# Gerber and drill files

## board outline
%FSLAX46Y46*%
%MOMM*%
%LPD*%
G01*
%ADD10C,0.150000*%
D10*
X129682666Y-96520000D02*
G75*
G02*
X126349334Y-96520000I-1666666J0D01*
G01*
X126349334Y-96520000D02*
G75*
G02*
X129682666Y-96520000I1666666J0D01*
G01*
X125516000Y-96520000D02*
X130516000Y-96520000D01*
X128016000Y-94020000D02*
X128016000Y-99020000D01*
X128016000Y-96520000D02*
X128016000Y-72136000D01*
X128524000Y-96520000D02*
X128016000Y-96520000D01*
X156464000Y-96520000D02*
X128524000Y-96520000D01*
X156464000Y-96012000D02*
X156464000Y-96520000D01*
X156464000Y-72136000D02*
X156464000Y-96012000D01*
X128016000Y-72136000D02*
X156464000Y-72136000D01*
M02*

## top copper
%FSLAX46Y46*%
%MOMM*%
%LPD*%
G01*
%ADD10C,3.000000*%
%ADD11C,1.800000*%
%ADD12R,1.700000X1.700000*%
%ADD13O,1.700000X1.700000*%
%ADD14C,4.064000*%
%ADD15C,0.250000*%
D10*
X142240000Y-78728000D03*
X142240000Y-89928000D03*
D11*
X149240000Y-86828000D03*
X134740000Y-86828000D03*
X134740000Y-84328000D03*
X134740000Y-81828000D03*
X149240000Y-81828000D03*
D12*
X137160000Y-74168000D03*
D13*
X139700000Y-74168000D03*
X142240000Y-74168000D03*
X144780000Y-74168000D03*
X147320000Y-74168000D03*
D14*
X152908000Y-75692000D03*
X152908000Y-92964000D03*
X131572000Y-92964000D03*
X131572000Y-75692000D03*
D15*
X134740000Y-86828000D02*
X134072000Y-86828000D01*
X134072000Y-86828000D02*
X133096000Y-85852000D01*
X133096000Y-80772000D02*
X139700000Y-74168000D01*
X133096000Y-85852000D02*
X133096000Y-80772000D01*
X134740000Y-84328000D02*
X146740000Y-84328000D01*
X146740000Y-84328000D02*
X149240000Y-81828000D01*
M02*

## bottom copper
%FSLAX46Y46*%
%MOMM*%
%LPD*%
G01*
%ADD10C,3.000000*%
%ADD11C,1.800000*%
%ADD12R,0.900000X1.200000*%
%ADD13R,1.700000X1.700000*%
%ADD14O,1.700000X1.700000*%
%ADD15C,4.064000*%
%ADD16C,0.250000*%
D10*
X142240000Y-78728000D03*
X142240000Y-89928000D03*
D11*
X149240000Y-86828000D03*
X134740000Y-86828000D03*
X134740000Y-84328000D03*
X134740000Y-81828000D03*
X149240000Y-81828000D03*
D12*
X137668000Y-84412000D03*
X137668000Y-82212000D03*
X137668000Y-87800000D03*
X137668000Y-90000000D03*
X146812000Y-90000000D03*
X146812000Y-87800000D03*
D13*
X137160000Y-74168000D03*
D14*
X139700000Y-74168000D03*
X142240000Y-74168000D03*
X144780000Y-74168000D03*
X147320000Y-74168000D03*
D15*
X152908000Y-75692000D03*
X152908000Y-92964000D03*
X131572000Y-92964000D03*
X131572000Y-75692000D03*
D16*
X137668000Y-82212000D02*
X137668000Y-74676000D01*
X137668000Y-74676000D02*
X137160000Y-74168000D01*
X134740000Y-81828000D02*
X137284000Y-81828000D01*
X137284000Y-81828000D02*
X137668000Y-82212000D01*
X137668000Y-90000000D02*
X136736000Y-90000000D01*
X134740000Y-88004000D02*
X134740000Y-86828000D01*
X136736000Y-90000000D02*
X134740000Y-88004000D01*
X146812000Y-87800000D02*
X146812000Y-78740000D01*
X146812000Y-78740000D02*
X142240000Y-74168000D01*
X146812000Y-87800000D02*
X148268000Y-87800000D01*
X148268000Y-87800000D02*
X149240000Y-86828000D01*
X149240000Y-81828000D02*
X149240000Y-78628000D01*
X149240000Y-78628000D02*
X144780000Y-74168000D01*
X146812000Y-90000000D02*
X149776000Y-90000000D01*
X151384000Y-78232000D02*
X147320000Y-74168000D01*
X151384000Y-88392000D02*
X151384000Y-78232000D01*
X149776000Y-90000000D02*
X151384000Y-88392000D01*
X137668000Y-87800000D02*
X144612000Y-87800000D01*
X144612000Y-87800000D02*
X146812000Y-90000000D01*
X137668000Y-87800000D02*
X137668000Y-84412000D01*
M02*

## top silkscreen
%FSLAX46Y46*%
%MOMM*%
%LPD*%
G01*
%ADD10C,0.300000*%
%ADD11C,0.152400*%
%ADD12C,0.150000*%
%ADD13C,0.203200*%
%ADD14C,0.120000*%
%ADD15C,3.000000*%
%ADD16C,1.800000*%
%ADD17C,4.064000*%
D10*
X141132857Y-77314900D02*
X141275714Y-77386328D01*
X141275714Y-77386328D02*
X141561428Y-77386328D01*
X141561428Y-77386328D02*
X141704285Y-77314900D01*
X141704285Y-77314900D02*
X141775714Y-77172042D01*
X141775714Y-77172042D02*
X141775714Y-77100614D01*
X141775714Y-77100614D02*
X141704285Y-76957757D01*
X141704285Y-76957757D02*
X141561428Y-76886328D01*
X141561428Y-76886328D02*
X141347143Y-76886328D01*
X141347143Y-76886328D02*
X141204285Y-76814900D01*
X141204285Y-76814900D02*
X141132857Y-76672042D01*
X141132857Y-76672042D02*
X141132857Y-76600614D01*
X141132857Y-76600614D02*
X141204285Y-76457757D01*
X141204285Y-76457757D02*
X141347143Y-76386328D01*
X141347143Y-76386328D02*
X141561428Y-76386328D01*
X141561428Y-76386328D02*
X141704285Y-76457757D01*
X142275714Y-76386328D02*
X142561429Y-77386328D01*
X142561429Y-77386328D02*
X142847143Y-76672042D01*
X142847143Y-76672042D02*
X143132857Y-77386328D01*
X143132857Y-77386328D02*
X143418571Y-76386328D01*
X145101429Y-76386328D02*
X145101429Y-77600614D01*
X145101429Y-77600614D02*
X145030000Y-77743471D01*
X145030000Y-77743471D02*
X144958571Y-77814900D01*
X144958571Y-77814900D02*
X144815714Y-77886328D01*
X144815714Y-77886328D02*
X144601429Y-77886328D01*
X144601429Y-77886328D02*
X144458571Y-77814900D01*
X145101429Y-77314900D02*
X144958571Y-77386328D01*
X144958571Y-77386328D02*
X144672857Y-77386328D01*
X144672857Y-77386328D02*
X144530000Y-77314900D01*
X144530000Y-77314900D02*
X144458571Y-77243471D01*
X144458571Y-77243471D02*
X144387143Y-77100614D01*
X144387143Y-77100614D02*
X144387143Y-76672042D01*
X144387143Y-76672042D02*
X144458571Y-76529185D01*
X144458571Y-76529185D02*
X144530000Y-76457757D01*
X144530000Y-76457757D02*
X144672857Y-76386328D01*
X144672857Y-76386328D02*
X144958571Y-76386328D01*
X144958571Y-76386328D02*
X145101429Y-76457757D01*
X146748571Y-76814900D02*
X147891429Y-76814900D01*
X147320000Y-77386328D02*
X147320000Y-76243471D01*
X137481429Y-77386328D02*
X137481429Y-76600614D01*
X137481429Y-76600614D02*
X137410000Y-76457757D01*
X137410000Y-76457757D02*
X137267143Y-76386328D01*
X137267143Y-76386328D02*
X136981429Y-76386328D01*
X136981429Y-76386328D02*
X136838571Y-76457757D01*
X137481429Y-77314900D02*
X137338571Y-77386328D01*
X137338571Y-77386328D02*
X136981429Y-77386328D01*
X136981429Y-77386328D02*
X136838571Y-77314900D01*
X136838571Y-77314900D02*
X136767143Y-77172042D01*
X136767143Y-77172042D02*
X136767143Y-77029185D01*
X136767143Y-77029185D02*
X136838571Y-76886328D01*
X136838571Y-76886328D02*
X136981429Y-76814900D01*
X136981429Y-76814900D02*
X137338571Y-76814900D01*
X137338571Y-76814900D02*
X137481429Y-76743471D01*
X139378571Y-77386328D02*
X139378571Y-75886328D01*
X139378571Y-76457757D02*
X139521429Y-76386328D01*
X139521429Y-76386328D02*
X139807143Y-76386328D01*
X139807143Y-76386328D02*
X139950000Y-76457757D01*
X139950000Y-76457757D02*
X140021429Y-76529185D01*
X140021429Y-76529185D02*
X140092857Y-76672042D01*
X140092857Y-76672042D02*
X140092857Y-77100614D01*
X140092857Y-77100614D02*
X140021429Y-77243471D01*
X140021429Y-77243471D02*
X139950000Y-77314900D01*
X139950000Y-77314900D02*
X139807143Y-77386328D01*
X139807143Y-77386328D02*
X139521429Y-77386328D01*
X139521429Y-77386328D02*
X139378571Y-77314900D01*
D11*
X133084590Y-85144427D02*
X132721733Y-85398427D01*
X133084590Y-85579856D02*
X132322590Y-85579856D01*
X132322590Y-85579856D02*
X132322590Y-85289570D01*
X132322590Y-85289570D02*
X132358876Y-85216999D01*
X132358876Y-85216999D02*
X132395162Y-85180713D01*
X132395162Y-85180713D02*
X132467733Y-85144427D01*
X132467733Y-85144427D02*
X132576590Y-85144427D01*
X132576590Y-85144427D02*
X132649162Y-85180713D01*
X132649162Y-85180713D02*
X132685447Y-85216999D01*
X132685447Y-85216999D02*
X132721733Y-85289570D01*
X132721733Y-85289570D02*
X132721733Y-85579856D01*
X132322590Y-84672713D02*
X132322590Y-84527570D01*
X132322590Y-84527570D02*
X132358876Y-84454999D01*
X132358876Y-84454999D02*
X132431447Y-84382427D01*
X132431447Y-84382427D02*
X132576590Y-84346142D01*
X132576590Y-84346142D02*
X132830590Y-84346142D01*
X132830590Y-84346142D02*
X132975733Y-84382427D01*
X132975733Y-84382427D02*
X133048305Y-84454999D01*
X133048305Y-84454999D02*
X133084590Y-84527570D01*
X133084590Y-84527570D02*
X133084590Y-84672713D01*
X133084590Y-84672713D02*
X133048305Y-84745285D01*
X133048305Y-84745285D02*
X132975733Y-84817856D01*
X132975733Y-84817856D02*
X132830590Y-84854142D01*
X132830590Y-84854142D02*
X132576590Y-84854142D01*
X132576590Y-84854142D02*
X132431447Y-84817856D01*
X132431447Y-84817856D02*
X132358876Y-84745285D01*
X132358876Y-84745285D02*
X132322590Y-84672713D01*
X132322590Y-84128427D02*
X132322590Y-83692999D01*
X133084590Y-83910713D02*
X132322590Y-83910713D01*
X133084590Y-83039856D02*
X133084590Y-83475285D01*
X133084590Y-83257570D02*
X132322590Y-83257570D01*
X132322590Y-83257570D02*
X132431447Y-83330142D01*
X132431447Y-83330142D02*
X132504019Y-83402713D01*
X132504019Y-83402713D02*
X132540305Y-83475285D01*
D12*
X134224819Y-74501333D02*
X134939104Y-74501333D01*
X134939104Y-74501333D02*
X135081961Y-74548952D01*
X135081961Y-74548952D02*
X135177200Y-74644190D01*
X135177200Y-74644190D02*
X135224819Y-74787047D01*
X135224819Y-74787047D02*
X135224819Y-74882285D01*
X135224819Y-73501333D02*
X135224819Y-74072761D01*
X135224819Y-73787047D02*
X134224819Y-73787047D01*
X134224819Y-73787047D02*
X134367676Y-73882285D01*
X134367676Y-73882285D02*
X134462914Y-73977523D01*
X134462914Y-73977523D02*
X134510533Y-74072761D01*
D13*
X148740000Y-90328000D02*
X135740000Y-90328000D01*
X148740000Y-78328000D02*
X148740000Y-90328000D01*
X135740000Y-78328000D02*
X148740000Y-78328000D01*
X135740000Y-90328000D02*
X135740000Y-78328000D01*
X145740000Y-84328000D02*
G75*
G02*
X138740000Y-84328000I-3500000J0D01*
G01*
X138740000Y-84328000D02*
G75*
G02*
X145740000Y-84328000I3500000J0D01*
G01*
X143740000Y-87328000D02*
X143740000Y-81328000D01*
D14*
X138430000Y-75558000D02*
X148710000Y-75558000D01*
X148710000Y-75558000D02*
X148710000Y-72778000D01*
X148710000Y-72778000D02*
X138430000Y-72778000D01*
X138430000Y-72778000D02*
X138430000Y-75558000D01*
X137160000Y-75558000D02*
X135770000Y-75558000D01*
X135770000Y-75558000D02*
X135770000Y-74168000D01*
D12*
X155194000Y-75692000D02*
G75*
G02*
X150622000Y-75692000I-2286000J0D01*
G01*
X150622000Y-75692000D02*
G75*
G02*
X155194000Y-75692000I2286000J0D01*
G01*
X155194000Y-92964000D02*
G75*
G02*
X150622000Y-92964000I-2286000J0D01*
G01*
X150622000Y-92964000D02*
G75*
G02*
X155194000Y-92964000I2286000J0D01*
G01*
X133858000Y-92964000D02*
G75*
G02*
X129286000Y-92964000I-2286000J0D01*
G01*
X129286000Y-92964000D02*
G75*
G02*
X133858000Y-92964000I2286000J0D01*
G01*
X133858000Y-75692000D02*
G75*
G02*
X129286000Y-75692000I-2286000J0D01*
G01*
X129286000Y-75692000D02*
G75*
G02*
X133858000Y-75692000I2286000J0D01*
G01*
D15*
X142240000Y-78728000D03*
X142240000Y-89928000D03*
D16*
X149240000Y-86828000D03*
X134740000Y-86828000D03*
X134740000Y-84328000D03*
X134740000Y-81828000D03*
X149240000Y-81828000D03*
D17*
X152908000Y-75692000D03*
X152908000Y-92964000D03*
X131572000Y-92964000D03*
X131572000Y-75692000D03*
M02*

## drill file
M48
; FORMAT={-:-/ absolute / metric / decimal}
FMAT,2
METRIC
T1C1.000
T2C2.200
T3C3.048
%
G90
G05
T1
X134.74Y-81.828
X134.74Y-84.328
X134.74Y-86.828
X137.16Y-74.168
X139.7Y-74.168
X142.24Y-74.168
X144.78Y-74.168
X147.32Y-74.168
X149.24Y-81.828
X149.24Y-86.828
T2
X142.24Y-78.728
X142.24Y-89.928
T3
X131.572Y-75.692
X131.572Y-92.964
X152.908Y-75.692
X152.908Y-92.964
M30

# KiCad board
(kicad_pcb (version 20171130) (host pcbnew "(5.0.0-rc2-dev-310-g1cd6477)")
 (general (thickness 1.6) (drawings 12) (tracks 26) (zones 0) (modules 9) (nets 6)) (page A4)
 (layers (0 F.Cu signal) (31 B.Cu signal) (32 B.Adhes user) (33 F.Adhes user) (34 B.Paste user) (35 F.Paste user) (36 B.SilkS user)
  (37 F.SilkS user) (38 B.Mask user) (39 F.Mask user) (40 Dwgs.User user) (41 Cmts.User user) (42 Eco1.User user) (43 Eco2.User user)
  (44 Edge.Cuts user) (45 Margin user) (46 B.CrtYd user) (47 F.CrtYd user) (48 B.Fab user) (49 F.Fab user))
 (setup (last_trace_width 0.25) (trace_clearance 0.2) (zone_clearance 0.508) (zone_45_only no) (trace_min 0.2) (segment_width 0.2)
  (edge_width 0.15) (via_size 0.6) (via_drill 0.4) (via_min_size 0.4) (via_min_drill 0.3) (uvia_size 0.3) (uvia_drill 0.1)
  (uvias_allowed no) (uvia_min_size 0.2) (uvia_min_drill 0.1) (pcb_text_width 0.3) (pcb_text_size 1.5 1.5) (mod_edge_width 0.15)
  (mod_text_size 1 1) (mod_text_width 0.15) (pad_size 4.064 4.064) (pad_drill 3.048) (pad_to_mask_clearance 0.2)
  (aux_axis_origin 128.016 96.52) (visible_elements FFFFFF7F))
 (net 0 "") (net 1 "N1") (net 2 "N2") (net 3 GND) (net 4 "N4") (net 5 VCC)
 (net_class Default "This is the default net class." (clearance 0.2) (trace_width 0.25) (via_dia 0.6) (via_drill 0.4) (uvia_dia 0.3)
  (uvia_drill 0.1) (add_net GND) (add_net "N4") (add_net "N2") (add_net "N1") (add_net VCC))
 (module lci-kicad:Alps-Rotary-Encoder (layer F.Cu) (at 142.24 84.328 270)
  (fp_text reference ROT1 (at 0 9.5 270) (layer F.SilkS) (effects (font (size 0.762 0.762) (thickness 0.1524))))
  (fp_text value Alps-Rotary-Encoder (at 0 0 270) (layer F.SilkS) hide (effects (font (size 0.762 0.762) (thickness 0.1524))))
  (fp_line (start 6 -6.5) (end 6 6.5) (layer F.SilkS) (width 0.2032))
  (fp_line (start -6 -6.5) (end 6 -6.5) (layer F.SilkS) (width 0.2032))
  (fp_line (start -6 6.5) (end -6 -6.5) (layer F.SilkS) (width 0.2032))
  (fp_line (start 6 6.5) (end -6 6.5) (layer F.SilkS) (width 0.2032))
  (fp_circle (center 0 0) (end 3.5 0) (layer F.SilkS) (width 0.2032))
  (fp_line (start 3 -1.5) (end -3 -1.5) (layer F.SilkS) (width 0.2032))
  (pad "" thru_hole circle (at -5.6 0 270) (size 3 3) (drill 2.2) (layers *.Cu *.Mask F.SilkS))
  (pad "" thru_hole circle (at 5.6 0 270) (size 3 3) (drill 2.2) (layers *.Cu *.Mask F.SilkS))
  (pad 5 thru_hole circle (at 2.5 -7 270) (size 1.8 1.8) (drill 1) (layers *.Cu *.Mask F.SilkS) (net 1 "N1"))
  (pad 4 thru_hole circle (at 2.5 7.5 270) (size 1.8 1.8) (drill 1) (layers *.Cu *.Mask F.SilkS) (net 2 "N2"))
  (pad 3 thru_hole circle (at 0 7.5 270) (size 1.8 1.8) (drill 1) (layers *.Cu *.Mask F.SilkS) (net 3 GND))
  (pad 2 thru_hole circle (at -2.5 7.5 270) (size 1.8 1.8) (drill 1) (layers *.Cu *.Mask F.SilkS) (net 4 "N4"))
  (pad 1 thru_hole circle (at -2.5 -7 270) (size 1.8 1.8) (drill 1) (layers *.Cu *.Mask F.SilkS) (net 3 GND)))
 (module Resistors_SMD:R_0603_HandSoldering (layer B.Cu) (at 137.668 83.312 90)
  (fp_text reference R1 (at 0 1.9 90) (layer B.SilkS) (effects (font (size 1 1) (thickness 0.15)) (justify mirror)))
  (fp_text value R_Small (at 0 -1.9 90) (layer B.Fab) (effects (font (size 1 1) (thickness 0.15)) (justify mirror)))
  (pad 1 smd rect (at -1.1 0 90) (size 1.2 0.9) (layers B.Cu B.Paste B.Mask) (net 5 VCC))
  (pad 2 smd rect (at 1.1 0 90) (size 1.2 0.9) (layers B.Cu B.Paste B.Mask) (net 4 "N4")))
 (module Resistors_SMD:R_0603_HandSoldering (layer B.Cu) (at 137.668 88.9 270)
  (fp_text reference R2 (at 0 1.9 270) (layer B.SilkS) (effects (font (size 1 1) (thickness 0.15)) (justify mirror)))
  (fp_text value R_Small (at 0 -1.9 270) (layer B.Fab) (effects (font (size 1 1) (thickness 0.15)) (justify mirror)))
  (pad 1 smd rect (at -1.1 0 270) (size 1.2 0.9) (layers B.Cu B.Paste B.Mask) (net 5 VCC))
  (pad 2 smd rect (at 1.1 0 270) (size 1.2 0.9) (layers B.Cu B.Paste B.Mask) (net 2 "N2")))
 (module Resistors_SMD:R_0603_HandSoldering (layer B.Cu) (at 146.812 88.9 90)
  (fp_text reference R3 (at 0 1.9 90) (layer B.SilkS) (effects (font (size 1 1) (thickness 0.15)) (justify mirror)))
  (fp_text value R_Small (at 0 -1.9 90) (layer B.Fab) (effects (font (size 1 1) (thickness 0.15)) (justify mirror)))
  (pad 1 smd rect (at -1.1 0 90) (size 1.2 0.9) (layers B.Cu B.Paste B.Mask) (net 5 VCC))
  (pad 2 smd rect (at 1.1 0 90) (size 1.2 0.9) (layers B.Cu B.Paste B.Mask) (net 1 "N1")))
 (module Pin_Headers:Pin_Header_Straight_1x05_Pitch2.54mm (layer F.Cu) (at 137.16 74.168 90)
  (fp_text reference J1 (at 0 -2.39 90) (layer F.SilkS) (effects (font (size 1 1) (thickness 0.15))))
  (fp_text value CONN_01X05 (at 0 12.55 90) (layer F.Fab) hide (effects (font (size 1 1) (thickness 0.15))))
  (fp_line (start -1.39 1.27) (end -1.39 11.55) (layer F.SilkS) (width 0.12))
  (fp_line (start -1.39 11.55) (end 1.39 11.55) (layer F.SilkS) (width 0.12))
  (fp_line (start 1.39 11.55) (end 1.39 1.27) (layer F.SilkS) (width 0.12))
  (fp_line (start 1.39 1.27) (end -1.39 1.27) (layer F.SilkS) (width 0.12))
  (fp_line (start -1.39 0) (end -1.39 -1.39) (layer F.SilkS) (width 0.12))
  (fp_line (start -1.39 -1.39) (end 0 -1.39) (layer F.SilkS) (width 0.12))
  (pad 1 thru_hole rect (at 0 0 90) (size 1.7 1.7) (drill 1) (layers *.Cu *.Mask) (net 4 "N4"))
  (pad 2 thru_hole oval (at 0 2.54 90) (size 1.7 1.7) (drill 1) (layers *.Cu *.Mask) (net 2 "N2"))
  (pad 3 thru_hole oval (at 0 5.08 90) (size 1.7 1.7) (drill 1) (layers *.Cu *.Mask) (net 1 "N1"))
  (pad 4 thru_hole oval (at 0 7.62 90) (size 1.7 1.7) (drill 1) (layers *.Cu *.Mask) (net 3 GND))
  (pad 5 thru_hole oval (at 0 10.16 90) (size 1.7 1.7) (drill 1) (layers *.Cu *.Mask) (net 5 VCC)))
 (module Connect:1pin (layer F.Cu) (at 152.908 75.692)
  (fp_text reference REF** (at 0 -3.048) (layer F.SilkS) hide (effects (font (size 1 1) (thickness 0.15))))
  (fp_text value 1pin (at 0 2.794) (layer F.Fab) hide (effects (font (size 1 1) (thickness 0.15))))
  (fp_circle (center 0 0) (end 0 -2.286) (layer F.SilkS) (width 0.15))
  (pad 1 thru_hole circle (at 0 0) (size 4.064 4.064) (drill 3.048) (layers *.Cu *.Mask F.SilkS)))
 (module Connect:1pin (layer F.Cu) (at 152.908 92.964)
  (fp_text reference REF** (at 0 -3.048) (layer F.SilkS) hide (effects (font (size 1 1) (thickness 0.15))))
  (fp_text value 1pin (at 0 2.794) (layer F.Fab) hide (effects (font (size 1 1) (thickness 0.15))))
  (fp_circle (center 0 0) (end 0 -2.286) (layer F.SilkS) (width 0.15))
  (pad 1 thru_hole circle (at 0 0) (size 4.064 4.064) (drill 3.048) (layers *.Cu *.Mask F.SilkS)))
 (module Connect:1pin (layer F.Cu) (at 131.572 92.964)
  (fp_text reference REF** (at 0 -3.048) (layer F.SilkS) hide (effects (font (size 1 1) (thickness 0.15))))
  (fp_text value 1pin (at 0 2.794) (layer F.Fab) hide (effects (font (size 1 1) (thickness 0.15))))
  (fp_circle (center 0 0) (end 0 -2.286) (layer F.SilkS) (width 0.15))
  (pad 1 thru_hole circle (at 0 0) (size 4.064 4.064) (drill 3.048) (layers *.Cu *.Mask F.SilkS)))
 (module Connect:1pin (layer F.Cu) (at 131.572 75.692)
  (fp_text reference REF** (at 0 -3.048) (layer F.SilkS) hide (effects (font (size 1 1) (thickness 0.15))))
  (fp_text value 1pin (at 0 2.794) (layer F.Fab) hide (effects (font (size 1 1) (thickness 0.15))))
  (fp_circle (center 0 0) (end 0 -2.286) (layer F.SilkS) (width 0.15))
  (pad 1 thru_hole circle (at 0 0) (size 4.064 4.064) (drill 3.048) (layers *.Cu *.Mask F.SilkS)))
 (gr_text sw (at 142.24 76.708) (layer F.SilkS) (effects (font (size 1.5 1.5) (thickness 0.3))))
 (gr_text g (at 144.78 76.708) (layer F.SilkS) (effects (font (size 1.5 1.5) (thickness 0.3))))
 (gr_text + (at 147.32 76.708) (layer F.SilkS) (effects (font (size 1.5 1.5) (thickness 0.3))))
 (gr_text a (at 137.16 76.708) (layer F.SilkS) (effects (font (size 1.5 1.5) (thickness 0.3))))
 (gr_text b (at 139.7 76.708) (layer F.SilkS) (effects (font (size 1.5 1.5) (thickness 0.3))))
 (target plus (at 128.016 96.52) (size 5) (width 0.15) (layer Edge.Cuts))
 (gr_line (start 128.016 96.52) (end 128.016 72.136) (angle 90) (layer Edge.Cuts) (width 0.15))
 (gr_line (start 128.524 96.52) (end 128.016 96.52) (angle 90) (layer Edge.Cuts) (width 0.15))
 (gr_line (start 156.464 96.52) (end 128.524 96.52) (angle 90) (layer Edge.Cuts) (width 0.15))
 (gr_line (start 156.464 96.012) (end 156.464 96.52) (angle 90) (layer Edge.Cuts) (width 0.15))
 (gr_line (start 156.464 72.136) (end 156.464 96.012) (angle 90) (layer Edge.Cuts) (width 0.15))
 (gr_line (start 128.016 72.136) (end 156.464 72.136) (angle 90) (layer Edge.Cuts) (width 0.15))
 (segment (start 137.668 82.212) (end 137.668 74.676) (width 0.25) (layer B.Cu) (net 4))
 (segment (start 137.668 74.676) (end 137.16 74.168) (width 0.25) (layer B.Cu) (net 4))
 (segment (start 134.74 81.828) (end 137.284 81.828) (width 0.25) (layer B.Cu) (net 4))
 (segment (start 137.284 81.828) (end 137.668 82.212) (width 0.25) (layer B.Cu) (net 4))
 (segment (start 134.74 86.828) (end 134.072 86.828) (width 0.25) (layer F.Cu) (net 2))
 (segment (start 134.072 86.828) (end 133.096 85.852) (width 0.25) (layer F.Cu) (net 2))
 (segment (start 133.096 80.772) (end 139.7 74.168) (width 0.25) (layer F.Cu) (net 2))
 (segment (start 133.096 85.852) (end 133.096 80.772) (width 0.25) (layer F.Cu) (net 2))
 (segment (start 137.668 90) (end 136.736 90) (width 0.25) (layer B.Cu) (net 2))
 (segment (start 134.74 88.004) (end 134.74 86.828) (width 0.25) (layer B.Cu) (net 2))
 (segment (start 136.736 90) (end 134.74 88.004) (width 0.25) (layer B.Cu) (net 2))
 (segment (start 146.812 87.8) (end 146.812 78.74) (width 0.25) (layer B.Cu) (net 1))
 (segment (start 146.812 78.74) (end 142.24 74.168) (width 0.25) (layer B.Cu) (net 1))
 (segment (start 146.812 87.8) (end 148.268 87.8) (width 0.25) (layer B.Cu) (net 1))
 (segment (start 148.268 87.8) (end 149.24 86.828) (width 0.25) (layer B.Cu) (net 1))
 (segment (start 134.74 84.328) (end 146.74 84.328) (width 0.25) (layer F.Cu) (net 3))
 (segment (start 146.74 84.328) (end 149.24 81.828) (width 0.25) (layer F.Cu) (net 3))
 (segment (start 149.24 81.828) (end 149.24 78.628) (width 0.25) (layer B.Cu) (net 3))
 (segment (start 149.24 78.628) (end 144.78 74.168) (width 0.25) (layer B.Cu) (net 3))
 (segment (start 146.812 90) (end 149.776 90) (width 0.25) (layer B.Cu) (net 5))
 (segment (start 151.384 78.232) (end 147.32 74.168) (width 0.25) (layer B.Cu) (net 5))
 (segment (start 151.384 88.392) (end 151.384 78.232) (width 0.25) (layer B.Cu) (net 5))
 (segment (start 149.776 90) (end 151.384 88.392) (width 0.25) (layer B.Cu) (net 5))
 (segment (start 137.668 87.8) (end 144.612 87.8) (width 0.25) (layer B.Cu) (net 5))
 (segment (start 144.612 87.8) (end 146.812 90) (width 0.25) (layer B.Cu) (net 5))
 (segment (start 137.668 87.8) (end 137.668 84.412) (width 0.25) (layer B.Cu) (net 5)))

